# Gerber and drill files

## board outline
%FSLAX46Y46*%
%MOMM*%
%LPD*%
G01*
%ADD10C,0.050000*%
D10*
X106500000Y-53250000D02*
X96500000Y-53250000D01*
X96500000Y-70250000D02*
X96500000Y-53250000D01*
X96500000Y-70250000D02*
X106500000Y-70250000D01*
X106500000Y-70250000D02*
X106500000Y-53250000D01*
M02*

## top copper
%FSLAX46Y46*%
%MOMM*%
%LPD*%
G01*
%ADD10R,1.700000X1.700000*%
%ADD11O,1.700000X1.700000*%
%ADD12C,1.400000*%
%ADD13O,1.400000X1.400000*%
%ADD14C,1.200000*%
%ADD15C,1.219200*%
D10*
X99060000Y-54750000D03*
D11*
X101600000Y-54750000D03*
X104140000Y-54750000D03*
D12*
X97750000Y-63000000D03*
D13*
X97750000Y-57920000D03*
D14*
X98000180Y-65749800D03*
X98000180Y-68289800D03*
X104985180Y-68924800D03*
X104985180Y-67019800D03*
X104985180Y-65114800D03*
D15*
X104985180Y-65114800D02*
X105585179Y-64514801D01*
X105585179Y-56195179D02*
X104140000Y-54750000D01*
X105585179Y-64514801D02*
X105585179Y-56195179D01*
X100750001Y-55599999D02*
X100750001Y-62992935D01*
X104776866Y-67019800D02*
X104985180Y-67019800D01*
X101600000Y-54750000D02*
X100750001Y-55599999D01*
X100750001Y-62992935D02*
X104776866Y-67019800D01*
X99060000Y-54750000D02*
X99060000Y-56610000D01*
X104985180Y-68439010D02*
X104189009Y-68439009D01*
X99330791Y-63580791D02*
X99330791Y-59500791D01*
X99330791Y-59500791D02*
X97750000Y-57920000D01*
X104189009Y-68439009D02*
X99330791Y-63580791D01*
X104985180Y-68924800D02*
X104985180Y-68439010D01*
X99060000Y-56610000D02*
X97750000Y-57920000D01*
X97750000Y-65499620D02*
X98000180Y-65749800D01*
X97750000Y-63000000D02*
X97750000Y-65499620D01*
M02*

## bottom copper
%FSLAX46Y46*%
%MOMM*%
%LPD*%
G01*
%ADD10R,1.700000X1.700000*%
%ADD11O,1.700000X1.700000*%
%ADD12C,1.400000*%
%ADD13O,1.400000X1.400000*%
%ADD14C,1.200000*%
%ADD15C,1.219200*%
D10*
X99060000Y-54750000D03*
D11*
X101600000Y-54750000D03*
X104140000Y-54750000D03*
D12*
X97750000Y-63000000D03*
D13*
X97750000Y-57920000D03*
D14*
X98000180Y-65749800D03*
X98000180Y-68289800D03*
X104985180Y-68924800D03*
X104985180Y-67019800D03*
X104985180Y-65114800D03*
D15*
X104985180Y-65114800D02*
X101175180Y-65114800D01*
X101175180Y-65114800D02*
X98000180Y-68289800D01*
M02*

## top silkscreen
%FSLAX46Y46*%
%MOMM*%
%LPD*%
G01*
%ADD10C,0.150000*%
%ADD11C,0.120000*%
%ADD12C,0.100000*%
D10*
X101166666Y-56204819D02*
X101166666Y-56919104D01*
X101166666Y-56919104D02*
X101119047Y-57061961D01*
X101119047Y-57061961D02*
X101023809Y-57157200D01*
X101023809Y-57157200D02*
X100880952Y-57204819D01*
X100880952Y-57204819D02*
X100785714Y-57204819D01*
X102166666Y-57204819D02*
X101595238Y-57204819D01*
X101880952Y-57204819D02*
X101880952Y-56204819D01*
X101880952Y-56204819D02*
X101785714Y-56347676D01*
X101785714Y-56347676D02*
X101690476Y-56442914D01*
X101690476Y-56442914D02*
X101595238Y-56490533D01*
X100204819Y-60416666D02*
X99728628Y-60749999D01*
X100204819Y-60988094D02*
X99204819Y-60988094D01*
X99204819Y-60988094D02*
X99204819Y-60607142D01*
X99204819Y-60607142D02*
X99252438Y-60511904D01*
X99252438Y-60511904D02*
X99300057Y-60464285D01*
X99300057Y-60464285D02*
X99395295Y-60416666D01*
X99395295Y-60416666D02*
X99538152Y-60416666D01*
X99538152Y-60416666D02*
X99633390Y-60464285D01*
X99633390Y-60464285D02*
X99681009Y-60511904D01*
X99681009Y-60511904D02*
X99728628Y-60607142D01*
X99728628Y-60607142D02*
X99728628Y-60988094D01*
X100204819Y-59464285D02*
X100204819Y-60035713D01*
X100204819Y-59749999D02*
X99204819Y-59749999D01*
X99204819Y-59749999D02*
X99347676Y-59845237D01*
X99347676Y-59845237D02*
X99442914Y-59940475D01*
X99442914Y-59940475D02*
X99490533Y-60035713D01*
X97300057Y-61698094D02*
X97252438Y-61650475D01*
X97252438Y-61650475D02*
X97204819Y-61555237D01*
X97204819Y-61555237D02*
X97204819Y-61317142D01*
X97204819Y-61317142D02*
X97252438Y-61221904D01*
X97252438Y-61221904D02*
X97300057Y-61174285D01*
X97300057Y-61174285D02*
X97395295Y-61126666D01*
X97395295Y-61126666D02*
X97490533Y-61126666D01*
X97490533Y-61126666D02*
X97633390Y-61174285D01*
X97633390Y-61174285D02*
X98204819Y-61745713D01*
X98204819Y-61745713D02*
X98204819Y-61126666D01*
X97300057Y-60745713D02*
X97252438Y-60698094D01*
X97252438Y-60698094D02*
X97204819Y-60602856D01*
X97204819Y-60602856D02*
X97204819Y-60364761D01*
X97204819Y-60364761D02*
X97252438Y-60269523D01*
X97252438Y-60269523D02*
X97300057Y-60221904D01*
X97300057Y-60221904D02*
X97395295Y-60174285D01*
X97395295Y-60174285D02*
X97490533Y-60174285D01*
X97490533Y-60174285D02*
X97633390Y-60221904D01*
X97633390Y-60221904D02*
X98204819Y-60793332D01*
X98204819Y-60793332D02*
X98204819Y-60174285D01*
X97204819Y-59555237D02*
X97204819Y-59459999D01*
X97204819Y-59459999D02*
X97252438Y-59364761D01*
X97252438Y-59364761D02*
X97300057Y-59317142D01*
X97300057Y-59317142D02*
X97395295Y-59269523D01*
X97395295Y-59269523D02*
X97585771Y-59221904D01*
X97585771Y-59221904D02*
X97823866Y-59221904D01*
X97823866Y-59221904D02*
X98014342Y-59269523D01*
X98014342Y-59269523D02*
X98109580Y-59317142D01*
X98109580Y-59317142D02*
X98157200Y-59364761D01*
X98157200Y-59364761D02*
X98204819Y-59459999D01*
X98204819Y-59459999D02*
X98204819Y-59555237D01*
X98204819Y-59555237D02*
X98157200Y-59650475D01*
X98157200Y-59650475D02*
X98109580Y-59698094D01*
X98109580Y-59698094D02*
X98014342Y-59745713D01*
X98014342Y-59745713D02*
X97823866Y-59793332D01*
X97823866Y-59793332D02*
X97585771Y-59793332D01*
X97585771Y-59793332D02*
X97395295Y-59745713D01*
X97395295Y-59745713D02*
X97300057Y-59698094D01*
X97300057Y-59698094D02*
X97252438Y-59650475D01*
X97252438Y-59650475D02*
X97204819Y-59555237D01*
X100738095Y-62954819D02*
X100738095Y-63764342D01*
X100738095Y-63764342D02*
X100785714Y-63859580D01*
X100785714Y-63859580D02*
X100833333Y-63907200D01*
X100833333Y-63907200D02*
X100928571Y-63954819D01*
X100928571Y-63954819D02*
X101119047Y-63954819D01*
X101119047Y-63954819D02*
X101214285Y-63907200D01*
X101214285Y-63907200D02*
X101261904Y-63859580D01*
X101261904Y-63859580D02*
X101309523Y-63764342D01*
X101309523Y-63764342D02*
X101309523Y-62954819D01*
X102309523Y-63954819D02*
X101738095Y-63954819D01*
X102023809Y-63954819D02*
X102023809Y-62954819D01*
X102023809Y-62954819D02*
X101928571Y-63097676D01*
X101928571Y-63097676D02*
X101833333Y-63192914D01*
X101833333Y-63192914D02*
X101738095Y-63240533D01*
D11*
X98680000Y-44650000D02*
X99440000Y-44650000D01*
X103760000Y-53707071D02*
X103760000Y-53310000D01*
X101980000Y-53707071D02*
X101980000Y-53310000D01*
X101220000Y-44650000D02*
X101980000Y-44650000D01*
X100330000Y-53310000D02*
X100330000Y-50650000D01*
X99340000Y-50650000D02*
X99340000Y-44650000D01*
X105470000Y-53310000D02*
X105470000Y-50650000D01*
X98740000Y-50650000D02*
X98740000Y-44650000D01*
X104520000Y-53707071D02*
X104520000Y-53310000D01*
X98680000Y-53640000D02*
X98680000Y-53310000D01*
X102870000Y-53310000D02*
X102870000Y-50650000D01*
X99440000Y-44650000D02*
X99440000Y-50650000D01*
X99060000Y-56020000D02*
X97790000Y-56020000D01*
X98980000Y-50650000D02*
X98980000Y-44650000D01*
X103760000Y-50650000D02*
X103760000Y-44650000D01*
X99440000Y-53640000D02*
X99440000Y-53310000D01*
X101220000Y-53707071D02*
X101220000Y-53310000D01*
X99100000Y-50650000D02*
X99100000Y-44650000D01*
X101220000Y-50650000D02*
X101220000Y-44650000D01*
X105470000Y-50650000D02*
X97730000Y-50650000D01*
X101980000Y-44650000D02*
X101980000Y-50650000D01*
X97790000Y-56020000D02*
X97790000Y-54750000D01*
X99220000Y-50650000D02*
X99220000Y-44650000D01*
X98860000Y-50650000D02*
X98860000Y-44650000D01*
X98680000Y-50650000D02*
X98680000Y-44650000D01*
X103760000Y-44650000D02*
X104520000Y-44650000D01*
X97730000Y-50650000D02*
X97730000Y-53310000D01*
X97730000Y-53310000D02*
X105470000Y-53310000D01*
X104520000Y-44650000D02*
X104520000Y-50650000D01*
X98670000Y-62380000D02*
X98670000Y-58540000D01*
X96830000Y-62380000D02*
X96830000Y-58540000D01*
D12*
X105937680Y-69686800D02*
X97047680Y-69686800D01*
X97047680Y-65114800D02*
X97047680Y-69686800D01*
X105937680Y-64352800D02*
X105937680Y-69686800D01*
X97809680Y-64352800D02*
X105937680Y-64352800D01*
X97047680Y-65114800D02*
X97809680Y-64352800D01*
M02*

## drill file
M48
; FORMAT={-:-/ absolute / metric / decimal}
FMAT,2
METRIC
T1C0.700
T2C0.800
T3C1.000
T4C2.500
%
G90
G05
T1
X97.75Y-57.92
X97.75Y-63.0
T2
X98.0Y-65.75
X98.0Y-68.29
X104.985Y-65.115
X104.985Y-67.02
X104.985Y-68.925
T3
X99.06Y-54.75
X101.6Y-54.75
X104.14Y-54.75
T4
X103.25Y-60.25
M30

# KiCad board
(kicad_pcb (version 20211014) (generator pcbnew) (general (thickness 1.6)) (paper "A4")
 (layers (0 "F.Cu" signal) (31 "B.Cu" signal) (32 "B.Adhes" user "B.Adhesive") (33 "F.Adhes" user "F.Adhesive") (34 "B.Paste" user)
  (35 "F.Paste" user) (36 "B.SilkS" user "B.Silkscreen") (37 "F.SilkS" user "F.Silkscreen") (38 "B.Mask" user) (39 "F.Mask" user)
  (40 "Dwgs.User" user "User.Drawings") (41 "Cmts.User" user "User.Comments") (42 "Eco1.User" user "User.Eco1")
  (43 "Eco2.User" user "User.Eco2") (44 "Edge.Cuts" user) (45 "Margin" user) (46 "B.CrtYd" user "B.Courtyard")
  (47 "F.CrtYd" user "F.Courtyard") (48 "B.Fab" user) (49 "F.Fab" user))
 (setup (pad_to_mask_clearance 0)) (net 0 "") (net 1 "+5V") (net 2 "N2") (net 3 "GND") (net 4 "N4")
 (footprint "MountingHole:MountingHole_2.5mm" (layer "F.Cu") (at 103.25 60.25)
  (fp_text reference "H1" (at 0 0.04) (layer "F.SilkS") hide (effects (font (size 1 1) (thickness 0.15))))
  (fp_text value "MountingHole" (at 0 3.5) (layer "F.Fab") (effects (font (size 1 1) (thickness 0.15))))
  (pad "" np_thru_hole circle locked (at 0 0) (size 2.5 2.5) (drill 2.5) (layers *.Cu *.Mask)))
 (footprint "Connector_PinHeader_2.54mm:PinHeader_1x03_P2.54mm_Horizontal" (layer "F.Cu") (at 99.06 54.75 90)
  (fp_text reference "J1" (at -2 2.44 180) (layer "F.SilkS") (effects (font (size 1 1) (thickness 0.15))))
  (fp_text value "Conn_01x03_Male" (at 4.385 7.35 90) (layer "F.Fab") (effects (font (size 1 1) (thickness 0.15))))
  (fp_line (start 10.1 -0.38) (end 10.1 0.38) (layer "F.SilkS") (width 0.12))
  (fp_line (start 1.042929 4.7) (end 1.44 4.7) (layer "F.SilkS") (width 0.12))
  (fp_line (start 1.042929 2.92) (end 1.44 2.92) (layer "F.SilkS") (width 0.12))
  (fp_line (start 10.1 2.16) (end 10.1 2.92) (layer "F.SilkS") (width 0.12))
  (fp_line (start 1.44 1.27) (end 4.1 1.27) (layer "F.SilkS") (width 0.12))
  (fp_line (start 4.1 0.28) (end 10.1 0.28) (layer "F.SilkS") (width 0.12))
  (fp_line (start 1.44 6.41) (end 4.1 6.41) (layer "F.SilkS") (width 0.12))
  (fp_line (start 4.1 -0.32) (end 10.1 -0.32) (layer "F.SilkS") (width 0.12))
  (fp_line (start 1.042929 5.46) (end 1.44 5.46) (layer "F.SilkS") (width 0.12))
  (fp_line (start 1.11 -0.38) (end 1.44 -0.38) (layer "F.SilkS") (width 0.12))
  (fp_line (start 1.44 3.81) (end 4.1 3.81) (layer "F.SilkS") (width 0.12))
  (fp_line (start 10.1 0.38) (end 4.1 0.38) (layer "F.SilkS") (width 0.12))
  (fp_line (start -1.27 0) (end -1.27 -1.27) (layer "F.SilkS") (width 0.12))
  (fp_line (start 4.1 -0.08) (end 10.1 -0.08) (layer "F.SilkS") (width 0.12))
  (fp_line (start 4.1 4.7) (end 10.1 4.7) (layer "F.SilkS") (width 0.12))
  (fp_line (start 1.11 0.38) (end 1.44 0.38) (layer "F.SilkS") (width 0.12))
  (fp_line (start 1.042929 2.16) (end 1.44 2.16) (layer "F.SilkS") (width 0.12))
  (fp_line (start 4.1 0.04) (end 10.1 0.04) (layer "F.SilkS") (width 0.12))
  (fp_line (start 4.1 2.16) (end 10.1 2.16) (layer "F.SilkS") (width 0.12))
  (fp_line (start 4.1 6.41) (end 4.1 -1.33) (layer "F.SilkS") (width 0.12))
  (fp_line (start 10.1 2.92) (end 4.1 2.92) (layer "F.SilkS") (width 0.12))
  (fp_line (start -1.27 -1.27) (end 0 -1.27) (layer "F.SilkS") (width 0.12))
  (fp_line (start 4.1 0.16) (end 10.1 0.16) (layer "F.SilkS") (width 0.12))
  (fp_line (start 4.1 -0.2) (end 10.1 -0.2) (layer "F.SilkS") (width 0.12))
  (fp_line (start 4.1 -0.38) (end 10.1 -0.38) (layer "F.SilkS") (width 0.12))
  (fp_line (start 10.1 4.7) (end 10.1 5.46) (layer "F.SilkS") (width 0.12))
  (fp_line (start 4.1 -1.33) (end 1.44 -1.33) (layer "F.SilkS") (width 0.12))
  (fp_line (start 1.44 -1.33) (end 1.44 6.41) (layer "F.SilkS") (width 0.12))
  (fp_line (start 10.1 5.46) (end 4.1 5.46) (layer "F.SilkS") (width 0.12))
  (pad "1" thru_hole rect locked (at 0 0 90) (size 1.7 1.7) (drill 1) (layers *.Cu *.Mask) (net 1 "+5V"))
  (pad "2" thru_hole oval locked (at 0 2.54 90) (size 1.7 1.7) (drill 1) (layers *.Cu *.Mask) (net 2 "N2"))
  (pad "3" thru_hole oval locked (at 0 5.08 90) (size 1.7 1.7) (drill 1) (layers *.Cu *.Mask) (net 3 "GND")))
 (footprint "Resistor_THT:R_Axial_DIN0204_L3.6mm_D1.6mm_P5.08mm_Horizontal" (layer "F.Cu") (at 97.75 63 90)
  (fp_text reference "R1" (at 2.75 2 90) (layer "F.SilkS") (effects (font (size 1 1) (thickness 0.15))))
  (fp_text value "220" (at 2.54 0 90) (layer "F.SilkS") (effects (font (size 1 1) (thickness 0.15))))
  (fp_line (start 0.62 0.92) (end 4.46 0.92) (layer "F.SilkS") (width 0.12))
  (fp_line (start 0.62 -0.92) (end 4.46 -0.92) (layer "F.SilkS") (width 0.12))
  (pad "1" thru_hole circle locked (at 0 0 90) (size 1.4 1.4) (drill 0.7) (layers *.Cu *.Mask) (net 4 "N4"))
  (pad "2" thru_hole oval locked (at 5.08 0 90) (size 1.4 1.4) (drill 0.7) (layers *.Cu *.Mask) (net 1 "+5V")))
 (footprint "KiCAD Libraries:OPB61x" (layer "F.Cu") (at 98 65.75)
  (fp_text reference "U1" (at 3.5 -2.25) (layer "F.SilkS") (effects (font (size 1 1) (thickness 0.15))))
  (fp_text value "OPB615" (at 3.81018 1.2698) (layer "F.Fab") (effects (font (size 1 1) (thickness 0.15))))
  (fp_line (start 7.93768 3.9368) (end -0.95232 3.9368) (layer "F.SilkS") (width 0.1))
  (fp_line (start -0.95232 -0.6352) (end -0.95232 3.9368) (layer "F.SilkS") (width 0.1))
  (fp_line (start 7.93768 -1.3972) (end 7.93768 3.9368) (layer "F.SilkS") (width 0.1))
  (fp_line (start -0.19032 -1.3972) (end 7.93768 -1.3972) (layer "F.SilkS") (width 0.1))
  (fp_line (start -0.95232 -0.6352) (end -0.19032 -1.3972) (layer "F.SilkS") (width 0.1))
  (pad "1" thru_hole circle locked (at 0.00018 -0.0002) (size 1.2 1.2) (drill 0.8) (layers *.Cu *.Mask) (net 4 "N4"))
  (pad "2" thru_hole circle locked (at 0.00018 2.5398) (size 1.2 1.2) (drill 0.8) (layers *.Cu *.Mask) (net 3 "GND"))
  (pad "3" thru_hole circle locked (at 6.98518 3.1748) (size 1.2 1.2) (drill 0.8) (layers *.Cu *.Mask) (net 1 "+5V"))
  (pad "4" thru_hole circle locked (at 6.98518 1.2698) (size 1.2 1.2) (drill 0.8) (layers *.Cu *.Mask) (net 2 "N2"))
  (pad "5" thru_hole circle locked (at 6.98518 -0.6352) (size 1.2 1.2) (drill 0.8) (layers *.Cu *.Mask) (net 3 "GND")))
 (gr_line (start 106.5 53.25) (end 96.5 53.25) (layer "Edge.Cuts") (width 0.05))
 (gr_line (start 96.5 70.25) (end 96.5 53.25) (layer "Edge.Cuts") (width 0.05))
 (gr_line (start 96.5 70.25) (end 106.5 70.25) (layer "Edge.Cuts") (width 0.05))
 (gr_line (start 106.5 70.25) (end 106.5 53.25) (layer "Edge.Cuts") (width 0.05))
 (segment (start 104.98518 65.1148) (end 105.585179 64.514801) (width 1.2192) (layer "F.Cu") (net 3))
 (segment (start 105.585179 56.195179) (end 104.14 54.75) (width 1.2192) (layer "F.Cu") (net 3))
 (segment (start 105.585179 64.514801) (end 105.585179 56.195179) (width 1.2192) (layer "F.Cu") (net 3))
 (segment (start 104.98518 65.1148) (end 101.17518 65.1148) (width 1.2192) (layer "B.Cu") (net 3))
 (segment (start 101.17518 65.1148) (end 98.00018 68.2898) (width 1.2192) (layer "B.Cu") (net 3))
 (segment (start 100.750001 55.599999) (end 100.750001 62.992935) (width 1.2192) (layer "F.Cu") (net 2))
 (segment (start 104.776866 67.0198) (end 104.98518 67.0198) (width 1.2192) (layer "F.Cu") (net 2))
 (segment (start 101.6 54.75) (end 100.750001 55.599999) (width 1.2192) (layer "F.Cu") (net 2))
 (segment (start 100.750001 62.992935) (end 104.776866 67.0198) (width 1.2192) (layer "F.Cu") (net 2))
 (segment (start 99.06 54.75) (end 99.06 56.61) (width 1.2192) (layer "F.Cu") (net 1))
 (segment (start 104.98518 68.43901) (end 104.189009 68.439009) (width 1.2192) (layer "F.Cu") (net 1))
 (segment (start 99.330791 63.580791) (end 99.330791 59.500791) (width 1.2192) (layer "F.Cu") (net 1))
 (segment (start 99.330791 59.500791) (end 97.75 57.92) (width 1.2192) (layer "F.Cu") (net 1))
 (segment (start 104.189009 68.439009) (end 99.330791 63.580791) (width 1.2192) (layer "F.Cu") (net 1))
 (segment (start 104.98518 68.9248) (end 104.98518 68.43901) (width 1.2192) (layer "F.Cu") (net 1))
 (segment (start 99.06 56.61) (end 97.75 57.92) (width 1.2192) (layer "F.Cu") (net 1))
 (segment (start 97.75 65.49962) (end 98.00018 65.7498) (width 1.2192) (layer "F.Cu") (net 4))
 (segment (start 97.75 63) (end 97.75 65.49962) (width 1.2192) (layer "F.Cu") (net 4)))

